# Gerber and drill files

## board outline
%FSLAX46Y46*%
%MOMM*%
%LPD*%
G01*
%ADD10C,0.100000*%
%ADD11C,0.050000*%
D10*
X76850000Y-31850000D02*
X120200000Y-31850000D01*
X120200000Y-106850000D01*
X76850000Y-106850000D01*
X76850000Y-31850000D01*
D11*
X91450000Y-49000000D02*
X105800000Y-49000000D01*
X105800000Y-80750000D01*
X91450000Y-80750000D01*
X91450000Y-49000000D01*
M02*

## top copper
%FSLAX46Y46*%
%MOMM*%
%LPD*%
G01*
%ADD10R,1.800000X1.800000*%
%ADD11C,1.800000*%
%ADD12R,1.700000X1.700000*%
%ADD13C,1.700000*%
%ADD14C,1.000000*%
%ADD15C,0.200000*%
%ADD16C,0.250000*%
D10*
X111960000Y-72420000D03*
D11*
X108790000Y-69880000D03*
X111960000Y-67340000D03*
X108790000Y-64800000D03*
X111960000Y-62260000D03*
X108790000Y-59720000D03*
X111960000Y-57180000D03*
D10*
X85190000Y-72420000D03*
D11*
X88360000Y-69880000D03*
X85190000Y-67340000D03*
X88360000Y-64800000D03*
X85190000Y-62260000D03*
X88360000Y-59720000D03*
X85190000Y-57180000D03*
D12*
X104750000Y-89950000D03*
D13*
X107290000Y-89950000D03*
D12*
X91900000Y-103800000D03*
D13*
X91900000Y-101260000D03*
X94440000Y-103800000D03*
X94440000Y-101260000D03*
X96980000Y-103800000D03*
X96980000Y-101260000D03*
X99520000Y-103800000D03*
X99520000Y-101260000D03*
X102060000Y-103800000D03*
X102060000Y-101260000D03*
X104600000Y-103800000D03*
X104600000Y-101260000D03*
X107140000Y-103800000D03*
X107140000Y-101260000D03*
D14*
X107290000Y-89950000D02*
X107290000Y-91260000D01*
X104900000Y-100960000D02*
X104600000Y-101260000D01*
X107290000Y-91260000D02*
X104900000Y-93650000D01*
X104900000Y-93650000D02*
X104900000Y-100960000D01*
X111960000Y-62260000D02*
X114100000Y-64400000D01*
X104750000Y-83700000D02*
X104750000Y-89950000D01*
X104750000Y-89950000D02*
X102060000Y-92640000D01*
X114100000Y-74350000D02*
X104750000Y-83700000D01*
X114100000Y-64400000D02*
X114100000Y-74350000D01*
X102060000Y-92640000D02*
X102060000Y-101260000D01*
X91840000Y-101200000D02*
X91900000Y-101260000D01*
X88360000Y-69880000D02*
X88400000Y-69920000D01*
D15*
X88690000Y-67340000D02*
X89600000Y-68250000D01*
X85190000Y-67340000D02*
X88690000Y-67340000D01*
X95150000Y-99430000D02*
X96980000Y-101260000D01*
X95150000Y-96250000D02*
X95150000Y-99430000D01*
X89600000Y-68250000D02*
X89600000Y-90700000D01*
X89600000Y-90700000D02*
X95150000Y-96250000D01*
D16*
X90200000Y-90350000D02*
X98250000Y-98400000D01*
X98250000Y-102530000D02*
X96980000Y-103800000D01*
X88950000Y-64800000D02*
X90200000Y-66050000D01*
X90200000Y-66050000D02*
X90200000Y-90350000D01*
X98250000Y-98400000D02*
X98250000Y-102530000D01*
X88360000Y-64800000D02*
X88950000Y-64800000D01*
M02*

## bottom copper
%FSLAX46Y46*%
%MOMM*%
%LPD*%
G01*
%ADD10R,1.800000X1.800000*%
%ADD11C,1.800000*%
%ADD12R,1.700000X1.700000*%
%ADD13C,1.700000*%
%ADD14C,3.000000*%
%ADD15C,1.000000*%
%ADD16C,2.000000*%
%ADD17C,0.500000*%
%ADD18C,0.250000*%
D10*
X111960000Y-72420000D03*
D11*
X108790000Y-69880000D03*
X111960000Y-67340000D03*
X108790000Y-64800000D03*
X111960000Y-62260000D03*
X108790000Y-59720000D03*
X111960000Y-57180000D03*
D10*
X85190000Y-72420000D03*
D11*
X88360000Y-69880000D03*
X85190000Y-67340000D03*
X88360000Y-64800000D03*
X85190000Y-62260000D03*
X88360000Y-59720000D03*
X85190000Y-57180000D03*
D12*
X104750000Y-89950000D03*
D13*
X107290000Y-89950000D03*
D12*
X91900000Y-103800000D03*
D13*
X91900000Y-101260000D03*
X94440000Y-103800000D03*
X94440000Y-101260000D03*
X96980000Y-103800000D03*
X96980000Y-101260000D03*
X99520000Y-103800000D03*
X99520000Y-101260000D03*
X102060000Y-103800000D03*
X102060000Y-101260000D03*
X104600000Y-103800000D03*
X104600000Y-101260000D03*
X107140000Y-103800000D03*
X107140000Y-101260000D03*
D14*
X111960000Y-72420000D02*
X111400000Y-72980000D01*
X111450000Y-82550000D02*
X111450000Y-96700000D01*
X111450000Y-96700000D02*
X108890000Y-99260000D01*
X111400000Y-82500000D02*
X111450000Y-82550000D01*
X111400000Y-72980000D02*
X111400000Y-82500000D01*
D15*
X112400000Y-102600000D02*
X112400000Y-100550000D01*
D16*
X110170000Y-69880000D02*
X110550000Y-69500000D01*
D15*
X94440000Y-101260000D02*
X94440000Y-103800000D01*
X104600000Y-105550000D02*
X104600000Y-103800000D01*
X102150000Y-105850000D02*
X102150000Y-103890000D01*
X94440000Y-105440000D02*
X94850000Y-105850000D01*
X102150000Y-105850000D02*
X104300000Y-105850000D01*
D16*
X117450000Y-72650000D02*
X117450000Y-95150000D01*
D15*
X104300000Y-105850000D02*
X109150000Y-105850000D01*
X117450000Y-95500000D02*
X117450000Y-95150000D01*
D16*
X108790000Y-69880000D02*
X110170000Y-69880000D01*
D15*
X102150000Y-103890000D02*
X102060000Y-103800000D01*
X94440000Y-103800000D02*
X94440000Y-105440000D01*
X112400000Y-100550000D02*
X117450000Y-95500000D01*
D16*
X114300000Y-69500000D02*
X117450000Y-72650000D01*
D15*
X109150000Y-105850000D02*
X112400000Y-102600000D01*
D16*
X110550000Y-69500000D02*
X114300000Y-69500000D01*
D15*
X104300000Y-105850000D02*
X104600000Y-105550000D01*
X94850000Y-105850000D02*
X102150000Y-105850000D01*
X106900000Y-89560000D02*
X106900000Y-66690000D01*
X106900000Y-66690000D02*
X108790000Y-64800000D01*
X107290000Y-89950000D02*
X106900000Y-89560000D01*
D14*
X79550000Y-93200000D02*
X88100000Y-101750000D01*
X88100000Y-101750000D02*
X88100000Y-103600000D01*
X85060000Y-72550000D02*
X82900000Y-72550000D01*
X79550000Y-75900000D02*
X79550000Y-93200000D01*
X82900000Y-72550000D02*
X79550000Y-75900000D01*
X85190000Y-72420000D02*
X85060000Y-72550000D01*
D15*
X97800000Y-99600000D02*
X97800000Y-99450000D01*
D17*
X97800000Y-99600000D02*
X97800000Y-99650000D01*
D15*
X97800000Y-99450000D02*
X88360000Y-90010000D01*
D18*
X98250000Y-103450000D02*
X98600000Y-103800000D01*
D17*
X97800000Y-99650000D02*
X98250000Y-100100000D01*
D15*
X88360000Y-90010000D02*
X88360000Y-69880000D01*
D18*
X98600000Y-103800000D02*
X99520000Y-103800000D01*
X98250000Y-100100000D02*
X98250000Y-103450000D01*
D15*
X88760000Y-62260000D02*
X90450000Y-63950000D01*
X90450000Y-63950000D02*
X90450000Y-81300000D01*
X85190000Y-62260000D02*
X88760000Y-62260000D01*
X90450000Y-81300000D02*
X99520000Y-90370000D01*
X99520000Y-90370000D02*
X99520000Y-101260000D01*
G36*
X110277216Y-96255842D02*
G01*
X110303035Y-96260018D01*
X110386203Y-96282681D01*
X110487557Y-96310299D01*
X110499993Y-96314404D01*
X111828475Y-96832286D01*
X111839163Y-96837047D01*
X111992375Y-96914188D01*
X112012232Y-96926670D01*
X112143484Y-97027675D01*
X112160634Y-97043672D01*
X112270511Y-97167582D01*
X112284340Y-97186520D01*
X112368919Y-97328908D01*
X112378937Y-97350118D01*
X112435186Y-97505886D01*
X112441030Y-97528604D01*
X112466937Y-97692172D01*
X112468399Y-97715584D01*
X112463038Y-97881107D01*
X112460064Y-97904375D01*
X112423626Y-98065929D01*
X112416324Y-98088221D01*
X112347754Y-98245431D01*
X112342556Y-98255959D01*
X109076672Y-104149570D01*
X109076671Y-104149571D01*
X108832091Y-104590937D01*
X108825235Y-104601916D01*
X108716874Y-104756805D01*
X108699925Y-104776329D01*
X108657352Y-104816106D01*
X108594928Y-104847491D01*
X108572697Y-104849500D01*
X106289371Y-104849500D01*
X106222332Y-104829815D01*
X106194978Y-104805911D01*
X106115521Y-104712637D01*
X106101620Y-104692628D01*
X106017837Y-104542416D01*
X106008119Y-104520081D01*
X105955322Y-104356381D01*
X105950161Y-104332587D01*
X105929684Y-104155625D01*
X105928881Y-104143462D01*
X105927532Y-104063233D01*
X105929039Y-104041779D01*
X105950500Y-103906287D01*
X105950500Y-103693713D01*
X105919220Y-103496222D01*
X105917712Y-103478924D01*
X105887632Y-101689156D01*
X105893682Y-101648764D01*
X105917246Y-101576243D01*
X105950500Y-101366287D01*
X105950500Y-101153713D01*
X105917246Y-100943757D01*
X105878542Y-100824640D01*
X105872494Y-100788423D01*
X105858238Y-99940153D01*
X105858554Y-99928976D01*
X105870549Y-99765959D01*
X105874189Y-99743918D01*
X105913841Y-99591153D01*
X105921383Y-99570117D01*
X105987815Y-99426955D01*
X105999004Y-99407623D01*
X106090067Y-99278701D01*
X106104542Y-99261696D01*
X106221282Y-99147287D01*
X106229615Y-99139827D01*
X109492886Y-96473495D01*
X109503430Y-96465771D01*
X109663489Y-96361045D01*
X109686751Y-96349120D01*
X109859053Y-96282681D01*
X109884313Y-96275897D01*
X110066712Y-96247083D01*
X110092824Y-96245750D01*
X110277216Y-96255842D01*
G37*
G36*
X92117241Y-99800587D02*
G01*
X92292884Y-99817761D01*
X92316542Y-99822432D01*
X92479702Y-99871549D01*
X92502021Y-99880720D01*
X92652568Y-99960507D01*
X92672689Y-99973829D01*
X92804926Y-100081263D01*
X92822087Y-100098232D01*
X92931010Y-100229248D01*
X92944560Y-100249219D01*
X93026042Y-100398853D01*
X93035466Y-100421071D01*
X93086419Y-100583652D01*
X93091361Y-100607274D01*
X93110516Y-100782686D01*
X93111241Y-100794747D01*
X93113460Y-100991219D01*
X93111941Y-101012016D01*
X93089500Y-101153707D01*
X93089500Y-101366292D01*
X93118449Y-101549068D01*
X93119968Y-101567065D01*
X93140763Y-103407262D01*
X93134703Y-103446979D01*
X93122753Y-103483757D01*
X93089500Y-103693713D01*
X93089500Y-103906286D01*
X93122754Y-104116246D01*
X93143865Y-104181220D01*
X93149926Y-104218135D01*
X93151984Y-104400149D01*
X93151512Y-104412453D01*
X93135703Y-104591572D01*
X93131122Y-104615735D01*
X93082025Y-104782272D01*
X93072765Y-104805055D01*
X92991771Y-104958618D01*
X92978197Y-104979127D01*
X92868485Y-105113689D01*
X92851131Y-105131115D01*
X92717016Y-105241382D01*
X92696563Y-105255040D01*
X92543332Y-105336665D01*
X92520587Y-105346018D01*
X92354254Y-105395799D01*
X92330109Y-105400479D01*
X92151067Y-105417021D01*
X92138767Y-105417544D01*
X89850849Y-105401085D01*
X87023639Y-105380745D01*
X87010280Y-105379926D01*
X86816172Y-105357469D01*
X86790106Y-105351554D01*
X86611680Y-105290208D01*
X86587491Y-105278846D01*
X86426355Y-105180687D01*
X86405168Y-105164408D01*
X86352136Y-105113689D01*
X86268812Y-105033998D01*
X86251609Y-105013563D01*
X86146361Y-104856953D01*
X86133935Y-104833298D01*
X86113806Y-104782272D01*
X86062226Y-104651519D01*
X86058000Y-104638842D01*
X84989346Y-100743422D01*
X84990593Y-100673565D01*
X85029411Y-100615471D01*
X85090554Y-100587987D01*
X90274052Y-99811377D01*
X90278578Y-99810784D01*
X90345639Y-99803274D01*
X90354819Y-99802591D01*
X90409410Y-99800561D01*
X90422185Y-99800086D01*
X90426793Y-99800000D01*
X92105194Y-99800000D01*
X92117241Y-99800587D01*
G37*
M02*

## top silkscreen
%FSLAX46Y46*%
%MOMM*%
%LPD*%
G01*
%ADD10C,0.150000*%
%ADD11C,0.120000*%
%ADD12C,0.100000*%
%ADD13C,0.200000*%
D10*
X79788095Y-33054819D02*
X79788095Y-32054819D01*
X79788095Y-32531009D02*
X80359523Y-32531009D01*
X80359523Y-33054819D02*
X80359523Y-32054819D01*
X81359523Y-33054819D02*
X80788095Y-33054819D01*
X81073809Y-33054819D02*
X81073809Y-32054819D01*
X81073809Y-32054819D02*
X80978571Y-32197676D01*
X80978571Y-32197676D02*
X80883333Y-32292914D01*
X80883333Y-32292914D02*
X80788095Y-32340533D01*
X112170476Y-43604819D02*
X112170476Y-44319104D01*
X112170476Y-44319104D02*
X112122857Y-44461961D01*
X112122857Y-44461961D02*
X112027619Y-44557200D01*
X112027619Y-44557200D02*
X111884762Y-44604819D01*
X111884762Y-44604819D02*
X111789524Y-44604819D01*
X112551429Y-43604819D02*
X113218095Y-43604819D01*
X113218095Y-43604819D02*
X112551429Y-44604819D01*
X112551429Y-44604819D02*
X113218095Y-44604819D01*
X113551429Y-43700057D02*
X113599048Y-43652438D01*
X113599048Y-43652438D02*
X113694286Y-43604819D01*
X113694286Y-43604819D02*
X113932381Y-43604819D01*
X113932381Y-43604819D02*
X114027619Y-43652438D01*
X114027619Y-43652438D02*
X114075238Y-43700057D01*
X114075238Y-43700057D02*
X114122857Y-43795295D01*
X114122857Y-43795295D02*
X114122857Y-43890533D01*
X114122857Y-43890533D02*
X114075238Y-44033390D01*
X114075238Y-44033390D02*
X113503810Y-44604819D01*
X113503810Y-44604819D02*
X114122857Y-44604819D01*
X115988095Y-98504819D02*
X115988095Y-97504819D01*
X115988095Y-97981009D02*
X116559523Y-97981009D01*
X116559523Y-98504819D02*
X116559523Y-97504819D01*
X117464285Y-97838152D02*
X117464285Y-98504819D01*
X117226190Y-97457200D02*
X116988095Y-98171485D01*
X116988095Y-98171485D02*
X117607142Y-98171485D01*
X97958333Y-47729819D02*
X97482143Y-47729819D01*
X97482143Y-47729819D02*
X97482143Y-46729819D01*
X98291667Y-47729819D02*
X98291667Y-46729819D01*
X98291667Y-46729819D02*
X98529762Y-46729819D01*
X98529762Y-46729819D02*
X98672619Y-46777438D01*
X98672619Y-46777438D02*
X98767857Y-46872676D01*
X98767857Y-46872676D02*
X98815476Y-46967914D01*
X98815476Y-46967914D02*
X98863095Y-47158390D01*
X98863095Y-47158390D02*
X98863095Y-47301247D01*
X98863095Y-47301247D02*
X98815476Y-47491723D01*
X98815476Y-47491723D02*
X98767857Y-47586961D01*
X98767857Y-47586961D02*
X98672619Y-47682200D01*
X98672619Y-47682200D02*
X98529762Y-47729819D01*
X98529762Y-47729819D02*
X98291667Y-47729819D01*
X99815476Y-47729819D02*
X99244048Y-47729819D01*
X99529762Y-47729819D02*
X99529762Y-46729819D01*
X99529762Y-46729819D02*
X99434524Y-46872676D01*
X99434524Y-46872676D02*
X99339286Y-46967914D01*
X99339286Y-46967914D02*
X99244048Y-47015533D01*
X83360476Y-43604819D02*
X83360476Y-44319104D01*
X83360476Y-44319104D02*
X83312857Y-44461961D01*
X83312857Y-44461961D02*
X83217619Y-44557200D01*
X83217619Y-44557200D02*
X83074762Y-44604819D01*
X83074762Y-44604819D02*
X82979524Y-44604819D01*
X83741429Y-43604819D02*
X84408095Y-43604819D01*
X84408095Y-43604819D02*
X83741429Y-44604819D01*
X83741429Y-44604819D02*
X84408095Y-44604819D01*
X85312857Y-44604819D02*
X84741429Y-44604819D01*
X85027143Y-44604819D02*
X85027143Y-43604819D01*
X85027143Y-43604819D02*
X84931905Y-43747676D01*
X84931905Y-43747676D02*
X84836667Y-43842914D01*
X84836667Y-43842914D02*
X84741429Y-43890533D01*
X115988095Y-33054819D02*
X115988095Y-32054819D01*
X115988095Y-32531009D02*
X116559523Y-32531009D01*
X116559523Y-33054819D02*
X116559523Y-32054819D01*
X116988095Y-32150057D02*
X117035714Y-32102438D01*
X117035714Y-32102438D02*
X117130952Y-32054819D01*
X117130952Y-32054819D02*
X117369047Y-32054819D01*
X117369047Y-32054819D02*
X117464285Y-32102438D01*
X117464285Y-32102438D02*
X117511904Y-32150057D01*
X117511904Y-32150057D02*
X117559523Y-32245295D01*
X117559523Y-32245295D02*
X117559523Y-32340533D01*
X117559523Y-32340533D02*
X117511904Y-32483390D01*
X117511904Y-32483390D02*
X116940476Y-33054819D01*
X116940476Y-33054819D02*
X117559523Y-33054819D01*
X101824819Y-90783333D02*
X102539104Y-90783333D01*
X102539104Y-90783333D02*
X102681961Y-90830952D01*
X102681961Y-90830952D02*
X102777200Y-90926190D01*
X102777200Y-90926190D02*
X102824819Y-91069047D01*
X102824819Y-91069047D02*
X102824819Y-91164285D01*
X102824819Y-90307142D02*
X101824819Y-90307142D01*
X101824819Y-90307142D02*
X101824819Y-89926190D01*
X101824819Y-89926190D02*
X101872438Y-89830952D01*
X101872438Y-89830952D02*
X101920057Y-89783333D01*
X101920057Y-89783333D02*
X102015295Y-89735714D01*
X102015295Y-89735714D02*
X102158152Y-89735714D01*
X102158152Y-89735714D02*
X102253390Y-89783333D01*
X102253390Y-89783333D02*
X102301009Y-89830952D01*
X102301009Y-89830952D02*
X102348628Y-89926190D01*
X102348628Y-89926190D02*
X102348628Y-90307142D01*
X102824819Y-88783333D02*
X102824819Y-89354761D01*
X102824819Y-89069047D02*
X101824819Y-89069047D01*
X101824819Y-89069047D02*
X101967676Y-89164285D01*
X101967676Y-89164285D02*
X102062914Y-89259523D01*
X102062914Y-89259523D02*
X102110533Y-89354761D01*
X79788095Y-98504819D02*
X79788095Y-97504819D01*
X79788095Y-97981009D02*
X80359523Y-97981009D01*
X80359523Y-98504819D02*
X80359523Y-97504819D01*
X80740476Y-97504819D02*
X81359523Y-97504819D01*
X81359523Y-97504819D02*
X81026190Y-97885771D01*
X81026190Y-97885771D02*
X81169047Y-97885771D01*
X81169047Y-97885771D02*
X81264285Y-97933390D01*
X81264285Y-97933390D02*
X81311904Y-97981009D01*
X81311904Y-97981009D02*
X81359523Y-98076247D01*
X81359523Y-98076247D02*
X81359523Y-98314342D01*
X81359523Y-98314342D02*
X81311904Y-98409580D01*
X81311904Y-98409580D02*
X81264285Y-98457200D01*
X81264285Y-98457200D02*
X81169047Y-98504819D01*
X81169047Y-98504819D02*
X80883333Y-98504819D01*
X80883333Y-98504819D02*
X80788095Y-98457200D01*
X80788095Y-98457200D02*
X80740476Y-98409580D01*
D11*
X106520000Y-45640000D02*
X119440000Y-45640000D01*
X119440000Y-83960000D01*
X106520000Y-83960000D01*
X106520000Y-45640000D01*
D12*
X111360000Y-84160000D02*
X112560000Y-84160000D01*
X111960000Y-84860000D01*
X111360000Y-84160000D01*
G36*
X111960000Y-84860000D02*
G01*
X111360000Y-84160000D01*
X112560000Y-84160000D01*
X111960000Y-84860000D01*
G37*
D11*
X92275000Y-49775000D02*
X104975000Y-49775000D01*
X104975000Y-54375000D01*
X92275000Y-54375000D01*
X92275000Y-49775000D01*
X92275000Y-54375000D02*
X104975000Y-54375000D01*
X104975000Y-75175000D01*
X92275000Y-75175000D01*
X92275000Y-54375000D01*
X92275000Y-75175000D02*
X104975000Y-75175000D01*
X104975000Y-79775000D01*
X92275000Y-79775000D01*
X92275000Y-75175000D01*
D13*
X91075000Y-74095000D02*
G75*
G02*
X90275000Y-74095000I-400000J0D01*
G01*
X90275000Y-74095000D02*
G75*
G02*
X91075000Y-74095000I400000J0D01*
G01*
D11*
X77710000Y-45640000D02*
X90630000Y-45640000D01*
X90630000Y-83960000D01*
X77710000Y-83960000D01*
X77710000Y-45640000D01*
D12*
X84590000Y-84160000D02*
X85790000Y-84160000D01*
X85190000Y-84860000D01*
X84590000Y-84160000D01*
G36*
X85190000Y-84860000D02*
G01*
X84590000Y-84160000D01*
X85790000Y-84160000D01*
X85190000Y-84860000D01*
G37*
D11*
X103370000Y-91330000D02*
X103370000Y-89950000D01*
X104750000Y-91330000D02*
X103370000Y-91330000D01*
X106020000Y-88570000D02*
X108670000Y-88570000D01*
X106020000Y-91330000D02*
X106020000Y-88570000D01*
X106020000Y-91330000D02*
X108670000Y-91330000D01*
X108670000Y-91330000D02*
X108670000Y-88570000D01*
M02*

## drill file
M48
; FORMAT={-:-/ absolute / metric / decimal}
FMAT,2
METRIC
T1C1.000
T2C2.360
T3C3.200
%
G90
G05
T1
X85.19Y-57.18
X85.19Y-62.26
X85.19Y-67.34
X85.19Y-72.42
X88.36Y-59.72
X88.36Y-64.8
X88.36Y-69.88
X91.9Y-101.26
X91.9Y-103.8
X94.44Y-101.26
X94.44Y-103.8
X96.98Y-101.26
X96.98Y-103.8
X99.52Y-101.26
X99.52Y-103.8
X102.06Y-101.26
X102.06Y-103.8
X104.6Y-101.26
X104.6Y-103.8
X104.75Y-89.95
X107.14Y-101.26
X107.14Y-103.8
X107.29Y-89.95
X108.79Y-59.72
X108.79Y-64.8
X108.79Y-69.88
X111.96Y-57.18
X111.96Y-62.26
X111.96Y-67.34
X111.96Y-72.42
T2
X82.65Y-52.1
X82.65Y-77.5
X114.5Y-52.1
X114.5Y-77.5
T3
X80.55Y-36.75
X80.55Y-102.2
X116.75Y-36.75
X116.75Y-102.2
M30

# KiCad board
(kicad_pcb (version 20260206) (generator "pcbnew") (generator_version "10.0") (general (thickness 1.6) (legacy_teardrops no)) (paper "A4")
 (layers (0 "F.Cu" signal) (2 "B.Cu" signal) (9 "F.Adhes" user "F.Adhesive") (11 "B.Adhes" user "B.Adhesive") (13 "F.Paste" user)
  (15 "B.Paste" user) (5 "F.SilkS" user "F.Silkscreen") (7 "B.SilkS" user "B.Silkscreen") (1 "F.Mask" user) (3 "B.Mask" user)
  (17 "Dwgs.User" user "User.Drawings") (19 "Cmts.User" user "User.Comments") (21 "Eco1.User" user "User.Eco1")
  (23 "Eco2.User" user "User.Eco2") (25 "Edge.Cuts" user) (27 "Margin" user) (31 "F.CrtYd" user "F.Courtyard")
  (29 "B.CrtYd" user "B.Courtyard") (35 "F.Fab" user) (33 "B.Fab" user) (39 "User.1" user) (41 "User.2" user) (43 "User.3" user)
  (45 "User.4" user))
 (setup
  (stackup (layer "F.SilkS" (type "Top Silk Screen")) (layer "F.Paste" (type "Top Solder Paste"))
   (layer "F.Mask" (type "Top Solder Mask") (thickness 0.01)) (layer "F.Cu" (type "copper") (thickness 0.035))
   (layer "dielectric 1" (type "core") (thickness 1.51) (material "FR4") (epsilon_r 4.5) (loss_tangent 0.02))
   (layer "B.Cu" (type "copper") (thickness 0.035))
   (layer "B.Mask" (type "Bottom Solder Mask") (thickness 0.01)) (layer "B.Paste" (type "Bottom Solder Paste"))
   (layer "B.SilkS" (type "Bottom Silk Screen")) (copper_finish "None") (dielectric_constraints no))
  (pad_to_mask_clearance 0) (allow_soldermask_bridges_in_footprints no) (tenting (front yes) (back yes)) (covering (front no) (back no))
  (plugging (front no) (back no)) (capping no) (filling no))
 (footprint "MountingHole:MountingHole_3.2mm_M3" (layer "F.Cu") (at 80.55 36.75)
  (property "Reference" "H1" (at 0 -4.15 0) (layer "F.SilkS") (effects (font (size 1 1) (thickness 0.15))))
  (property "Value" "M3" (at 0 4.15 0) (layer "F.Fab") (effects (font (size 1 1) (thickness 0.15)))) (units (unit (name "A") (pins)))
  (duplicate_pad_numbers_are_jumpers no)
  (pad "" np_thru_hole circle (at 0 0) (size 3.2 3.2) (drill 3.2) (layers "*.Cu" "*.Mask")))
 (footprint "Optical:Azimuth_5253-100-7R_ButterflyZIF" (layer "F.Cu") (at 112.98 64.8)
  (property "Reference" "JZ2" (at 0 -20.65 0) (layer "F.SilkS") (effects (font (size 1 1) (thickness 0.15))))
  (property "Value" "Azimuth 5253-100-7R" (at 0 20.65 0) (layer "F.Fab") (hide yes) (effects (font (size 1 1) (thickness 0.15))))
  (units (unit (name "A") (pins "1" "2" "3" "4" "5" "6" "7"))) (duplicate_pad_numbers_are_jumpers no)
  (fp_rect (start -6.46 -19.16) (end 6.46 19.16) (stroke (width 0.12) (type default)) (fill no) (layer "F.SilkS"))
  (fp_poly (pts (xy -1.62 19.36) (xy -0.42 19.36) (xy -1.02 20.06)) (stroke (width 0.1) (type default)) (fill yes) (layer "F.SilkS"))
  (pad "" np_thru_hole circle (at 1.52 -12.7) (size 2.36 2.36) (drill 2.36) (layers "*.Cu" "*.Mask"))
  (pad "" np_thru_hole circle (at 1.52 12.7) (size 2.36 2.36) (drill 2.36) (layers "*.Cu" "*.Mask"))
  (pad "1" thru_hole rect (at -1.02 7.62) (size 1.8 1.8) (drill 1) (layers "*.Cu" "*.Mask") (remove_unused_layers no) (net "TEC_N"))
  (pad "2" thru_hole circle (at -4.19 5.08) (size 1.8 1.8) (drill 1) (layers "*.Cu" "*.Mask") (remove_unused_layers no) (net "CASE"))
  (pad "3" thru_hole circle (at -1.02 2.54) (size 1.8 1.8) (drill 1) (layers "*.Cu" "*.Mask") (remove_unused_layers no)
   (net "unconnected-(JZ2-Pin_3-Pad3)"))
  (pad "4" thru_hole circle (at -4.19 0) (size 1.8 1.8) (drill 1) (layers "*.Cu" "*.Mask") (remove_unused_layers no) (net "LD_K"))
  (pad "5" thru_hole circle (at -1.02 -2.54) (size 1.8 1.8) (drill 1) (layers "*.Cu" "*.Mask") (remove_unused_layers no) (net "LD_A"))
  (pad "6" thru_hole circle (at -4.19 -5.08) (size 1.8 1.8) (drill 1) (layers "*.Cu" "*.Mask") (remove_unused_layers no)
   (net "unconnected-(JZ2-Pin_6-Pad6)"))
  (pad "7" thru_hole circle (at -1.02 -7.62) (size 1.8 1.8) (drill 1) (layers "*.Cu" "*.Mask") (remove_unused_layers no)
   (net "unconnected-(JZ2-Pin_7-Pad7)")))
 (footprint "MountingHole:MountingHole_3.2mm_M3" (layer "F.Cu") (at 116.75 102.2)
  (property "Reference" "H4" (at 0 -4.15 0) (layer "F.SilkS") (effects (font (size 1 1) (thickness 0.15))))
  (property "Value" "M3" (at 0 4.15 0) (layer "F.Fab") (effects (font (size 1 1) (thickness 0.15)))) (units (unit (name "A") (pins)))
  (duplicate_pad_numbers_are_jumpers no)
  (pad "" np_thru_hole circle (at 0 0) (size 3.2 3.2) (drill 3.2) (layers "*.Cu" "*.Mask")))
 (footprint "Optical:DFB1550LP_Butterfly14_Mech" (layer "F.Cu") (at 98.625 64.775)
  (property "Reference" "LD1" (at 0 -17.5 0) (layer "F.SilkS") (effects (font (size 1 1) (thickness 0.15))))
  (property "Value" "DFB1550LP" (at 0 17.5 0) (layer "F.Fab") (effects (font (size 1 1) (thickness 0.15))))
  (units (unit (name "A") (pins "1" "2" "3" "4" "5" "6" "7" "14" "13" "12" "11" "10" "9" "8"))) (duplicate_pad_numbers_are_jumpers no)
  (fp_rect (start -6.35 -15) (end 6.35 -10.4) (stroke (width 0.12) (type solid)) (fill no) (layer "F.SilkS"))
  (fp_rect (start -6.35 -10.4) (end 6.35 10.4) (stroke (width 0.12) (type solid)) (fill no) (layer "F.SilkS"))
  (fp_rect (start -6.35 10.4) (end 6.35 15) (stroke (width 0.12) (type solid)) (fill no) (layer "F.SilkS"))
  (fp_circle (center -7.95 9.32) (end -7.55 9.32) (stroke (width 0.2) (type solid)) (fill no) (layer "F.SilkS")))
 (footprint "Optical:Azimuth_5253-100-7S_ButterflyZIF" (layer "F.Cu") (at 84.17 64.8)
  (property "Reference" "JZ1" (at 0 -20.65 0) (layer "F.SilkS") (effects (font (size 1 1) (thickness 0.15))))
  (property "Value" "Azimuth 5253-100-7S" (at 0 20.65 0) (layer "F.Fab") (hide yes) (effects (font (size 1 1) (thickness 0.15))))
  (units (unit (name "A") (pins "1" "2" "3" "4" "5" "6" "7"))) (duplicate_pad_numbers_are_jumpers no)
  (fp_rect (start -6.46 -19.16) (end 6.46 19.16) (stroke (width 0.12) (type default)) (fill no) (layer "F.SilkS"))
  (fp_poly (pts (xy 0.42 19.36) (xy 1.62 19.36) (xy 1.02 20.06)) (stroke (width 0.1) (type default)) (fill yes) (layer "F.SilkS"))
  (pad "" np_thru_hole circle (at -1.52 -12.7) (size 2.36 2.36) (drill 2.36) (layers "*.Cu" "*.Mask"))
  (pad "" np_thru_hole circle (at -1.52 12.7) (size 2.36 2.36) (drill 2.36) (layers "*.Cu" "*.Mask"))
  (pad "1" thru_hole rect (at 1.02 7.62) (size 1.8 1.8) (drill 1) (layers "*.Cu" "*.Mask") (remove_unused_layers no) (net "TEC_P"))
  (pad "2" thru_hole circle (at 4.19 5.08) (size 1.8 1.8) (drill 1) (layers "*.Cu" "*.Mask") (remove_unused_layers no) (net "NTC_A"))
  (pad "3" thru_hole circle (at 1.02 2.54) (size 1.8 1.8) (drill 1) (layers "*.Cu" "*.Mask") (remove_unused_layers no) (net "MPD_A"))
  (pad "4" thru_hole circle (at 4.19 0) (size 1.8 1.8) (drill 1) (layers "*.Cu" "*.Mask") (remove_unused_layers no) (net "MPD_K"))
  (pad "5" thru_hole circle (at 1.02 -2.54) (size 1.8 1.8) (drill 1) (layers "*.Cu" "*.Mask") (remove_unused_layers no) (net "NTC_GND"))
  (pad "6" thru_hole circle (at 4.19 -5.08) (size 1.8 1.8) (drill 1) (layers "*.Cu" "*.Mask") (remove_unused_layers no)
   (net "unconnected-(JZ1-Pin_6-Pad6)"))
  (pad "7" thru_hole circle (at 1.02 -7.62) (size 1.8 1.8) (drill 1) (layers "*.Cu" "*.Mask") (remove_unused_layers no)
   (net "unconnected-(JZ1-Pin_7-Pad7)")))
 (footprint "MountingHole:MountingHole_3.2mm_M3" (layer "F.Cu") (at 116.75 36.75)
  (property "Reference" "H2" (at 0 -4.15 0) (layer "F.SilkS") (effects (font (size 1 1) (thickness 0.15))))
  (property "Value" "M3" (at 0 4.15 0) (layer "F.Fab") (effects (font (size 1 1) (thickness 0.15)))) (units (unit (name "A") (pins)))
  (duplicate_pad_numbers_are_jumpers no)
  (pad "" np_thru_hole circle (at 0 0) (size 3.2 3.2) (drill 3.2) (layers "*.Cu" "*.Mask")))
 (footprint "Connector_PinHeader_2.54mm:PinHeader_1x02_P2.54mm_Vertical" (layer "F.Cu") (at 104.75 89.95 90)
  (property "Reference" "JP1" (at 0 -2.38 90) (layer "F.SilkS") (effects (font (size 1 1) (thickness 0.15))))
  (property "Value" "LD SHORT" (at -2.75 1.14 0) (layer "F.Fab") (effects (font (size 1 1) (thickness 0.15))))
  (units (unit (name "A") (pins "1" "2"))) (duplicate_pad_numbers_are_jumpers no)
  (fp_line (start -1.38 -1.38) (end 0 -1.38) (stroke (width 0.12) (type solid)) (layer "F.SilkS"))
  (fp_line (start -1.38 0) (end -1.38 -1.38) (stroke (width 0.12) (type solid)) (layer "F.SilkS"))
  (fp_line (start 1.38 1.27) (end 1.38 3.92) (stroke (width 0.12) (type solid)) (layer "F.SilkS"))
  (fp_line (start -1.38 1.27) (end 1.38 1.27) (stroke (width 0.12) (type solid)) (layer "F.SilkS"))
  (fp_line (start -1.38 1.27) (end -1.38 3.92) (stroke (width 0.12) (type solid)) (layer "F.SilkS"))
  (fp_line (start -1.38 3.92) (end 1.38 3.92) (stroke (width 0.12) (type solid)) (layer "F.SilkS"))
  (pad "1" thru_hole rect (at 0 0 90) (size 1.7 1.7) (drill 1) (layers "*.Cu" "*.Mask") (remove_unused_layers no) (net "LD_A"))
  (pad "2" thru_hole circle (at 0 2.54 90) (size 1.7 1.7) (drill 1) (layers "*.Cu" "*.Mask") (remove_unused_layers no) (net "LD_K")))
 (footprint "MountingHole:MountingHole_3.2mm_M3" (layer "F.Cu") (at 80.55 102.2)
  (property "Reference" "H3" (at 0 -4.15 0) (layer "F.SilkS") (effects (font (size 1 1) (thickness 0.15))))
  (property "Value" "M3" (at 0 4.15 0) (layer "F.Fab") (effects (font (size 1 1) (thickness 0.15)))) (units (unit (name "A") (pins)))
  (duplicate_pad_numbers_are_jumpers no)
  (pad "" np_thru_hole circle (at 0 0) (size 3.2 3.2) (drill 3.2) (layers "*.Cu" "*.Mask")))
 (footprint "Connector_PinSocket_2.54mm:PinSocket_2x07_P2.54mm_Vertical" (layer "B.Cu") (at 91.9 103.8 -90)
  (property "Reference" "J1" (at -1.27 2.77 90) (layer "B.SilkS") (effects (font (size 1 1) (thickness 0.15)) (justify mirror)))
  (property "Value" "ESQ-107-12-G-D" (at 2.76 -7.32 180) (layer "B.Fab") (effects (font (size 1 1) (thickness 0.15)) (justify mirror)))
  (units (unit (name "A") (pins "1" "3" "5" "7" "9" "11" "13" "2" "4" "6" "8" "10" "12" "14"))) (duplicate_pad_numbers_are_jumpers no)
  (pad "1" thru_hole rect (at 0 0 270) (size 1.7 1.7) (drill 1) (layers "*.Cu" "*.Mask") (remove_unused_layers no) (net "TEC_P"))
  (pad "2" thru_hole circle (at -2.54 0 270) (size 1.7 1.7) (drill 1) (layers "*.Cu" "*.Mask") (remove_unused_layers no) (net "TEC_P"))
  (pad "3" thru_hole circle (at 0 -2.54 270) (size 1.7 1.7) (drill 1) (layers "*.Cu" "*.Mask") (remove_unused_layers no) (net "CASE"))
  (pad "4" thru_hole circle (at -2.54 -2.54 270) (size 1.7 1.7) (drill 1) (layers "*.Cu" "*.Mask") (remove_unused_layers no) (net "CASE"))
  (pad "5" thru_hole circle (at 0 -5.08 270) (size 1.7 1.7) (drill 1) (layers "*.Cu" "*.Mask") (remove_unused_layers no) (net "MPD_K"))
  (pad "6" thru_hole circle (at -2.54 -5.08 270) (size 1.7 1.7) (drill 1) (layers "*.Cu" "*.Mask") (remove_unused_layers no) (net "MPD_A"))
  (pad "7" thru_hole circle (at 0 -7.62 270) (size 1.7 1.7) (drill 1) (layers "*.Cu" "*.Mask") (remove_unused_layers no) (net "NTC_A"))
  (pad "8" thru_hole circle (at -2.54 -7.62 270) (size 1.7 1.7) (drill 1) (layers "*.Cu" "*.Mask") (remove_unused_layers no) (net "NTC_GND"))
  (pad "9" thru_hole circle (at 0 -10.16 270) (size 1.7 1.7) (drill 1) (layers "*.Cu" "*.Mask") (remove_unused_layers no) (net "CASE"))
  (pad "10" thru_hole circle (at -2.54 -10.16 270) (size 1.7 1.7) (drill 1) (layers "*.Cu" "*.Mask") (remove_unused_layers no) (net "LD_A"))
  (pad "11" thru_hole circle (at 0 -12.7 270) (size 1.7 1.7) (drill 1) (layers "*.Cu" "*.Mask") (remove_unused_layers no) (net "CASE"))
  (pad "12" thru_hole circle (at -2.54 -12.7 270) (size 1.7 1.7) (drill 1) (layers "*.Cu" "*.Mask") (remove_unused_layers no) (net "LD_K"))
  (pad "13" thru_hole circle (at 0 -15.24 270) (size 1.7 1.7) (drill 1) (layers "*.Cu" "*.Mask") (remove_unused_layers no) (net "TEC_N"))
  (pad "14" thru_hole circle (at -2.54 -15.24 270) (size 1.7 1.7) (drill 1) (layers "*.Cu" "*.Mask") (remove_unused_layers no) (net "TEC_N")))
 (gr_rect (start 76.85 31.85) (end 120.2 106.85) (stroke (width 0.1) (type solid)) (fill no) (layer "Edge.Cuts"))
 (gr_rect (start 91.45 49) (end 105.8 80.75) (stroke (width 0.05) (type default)) (fill no) (layer "Edge.Cuts"))
 (segment (start 111.96 72.42) (end 111.4 72.98) (width 3) (layer "B.Cu") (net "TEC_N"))
 (segment (start 111.45 82.55) (end 111.45 96.7) (width 3) (layer "B.Cu") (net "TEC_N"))
 (segment (start 111.45 96.7) (end 108.89 99.26) (width 3) (layer "B.Cu") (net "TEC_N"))
 (segment (start 111.4 82.5) (end 111.45 82.55) (width 3) (layer "B.Cu") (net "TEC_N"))
 (segment (start 111.4 72.98) (end 111.4 82.5) (width 3) (layer "B.Cu") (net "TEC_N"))
 (segment (start 112.4 102.6) (end 112.4 100.55) (width 1) (layer "B.Cu") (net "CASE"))
 (segment (start 110.17 69.88) (end 110.55 69.5) (width 2) (layer "B.Cu") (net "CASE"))
 (segment (start 94.44 101.26) (end 94.44 103.8) (width 1) (layer "B.Cu") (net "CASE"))
 (segment (start 104.6 105.55) (end 104.6 103.8) (width 1) (layer "B.Cu") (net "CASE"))
 (segment (start 102.15 105.85) (end 102.15 103.89) (width 1) (layer "B.Cu") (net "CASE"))
 (segment (start 94.44 105.44) (end 94.85 105.85) (width 1) (layer "B.Cu") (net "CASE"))
 (segment (start 102.15 105.85) (end 104.3 105.85) (width 1) (layer "B.Cu") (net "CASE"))
 (segment (start 117.45 72.65) (end 117.45 95.15) (width 2) (layer "B.Cu") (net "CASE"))
 (segment (start 104.3 105.85) (end 109.15 105.85) (width 1) (layer "B.Cu") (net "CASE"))
 (segment (start 117.45 95.5) (end 117.45 95.15) (width 1) (layer "B.Cu") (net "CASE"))
 (segment (start 108.79 69.88) (end 110.17 69.88) (width 2) (layer "B.Cu") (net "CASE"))
 (segment (start 102.15 103.89) (end 102.06 103.8) (width 1) (layer "B.Cu") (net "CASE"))
 (segment (start 94.44 103.8) (end 94.44 105.44) (width 1) (layer "B.Cu") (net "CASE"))
 (segment (start 112.4 100.55) (end 117.45 95.5) (width 1) (layer "B.Cu") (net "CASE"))
 (segment (start 114.3 69.5) (end 117.45 72.65) (width 2) (layer "B.Cu") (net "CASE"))
 (segment (start 109.15 105.85) (end 112.4 102.6) (width 1) (layer "B.Cu") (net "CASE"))
 (segment (start 110.55 69.5) (end 114.3 69.5) (width 2) (layer "B.Cu") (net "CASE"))
 (segment (start 104.3 105.85) (end 104.6 105.55) (width 1) (layer "B.Cu") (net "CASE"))
 (segment (start 94.85 105.85) (end 102.15 105.85) (width 1) (layer "B.Cu") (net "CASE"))
 (segment (start 107.29 89.95) (end 107.29 91.26) (width 1) (layer "F.Cu") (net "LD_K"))
 (segment (start 104.9 100.96) (end 104.6 101.26) (width 1) (layer "F.Cu") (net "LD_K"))
 (segment (start 107.29 91.26) (end 104.9 93.65) (width 1) (layer "F.Cu") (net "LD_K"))
 (segment (start 104.9 93.65) (end 104.9 100.96) (width 1) (layer "F.Cu") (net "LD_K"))
 (segment (start 106.9 89.56) (end 106.9 66.69) (width 1) (layer "B.Cu") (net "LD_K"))
 (segment (start 106.9 66.69) (end 108.79 64.8) (width 1) (layer "B.Cu") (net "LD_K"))
 (segment (start 107.29 89.95) (end 106.9 89.56) (width 1) (layer "B.Cu") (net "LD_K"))
 (segment (start 111.96 62.26) (end 114.1 64.4) (width 1) (layer "F.Cu") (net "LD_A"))
 (segment (start 104.75 83.7) (end 104.75 89.95) (width 1) (layer "F.Cu") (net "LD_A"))
 (segment (start 104.75 89.95) (end 102.06 92.64) (width 1) (layer "F.Cu") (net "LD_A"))
 (segment (start 114.1 74.35) (end 104.75 83.7) (width 1) (layer "F.Cu") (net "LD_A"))
 (segment (start 114.1 64.4) (end 114.1 74.35) (width 1) (layer "F.Cu") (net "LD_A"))
 (segment (start 102.06 92.64) (end 102.06 101.26) (width 1) (layer "F.Cu") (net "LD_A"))
 (segment (start 91.84 101.2) (end 91.9 101.26) (width 1) (layer "F.Cu") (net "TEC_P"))
 (segment (start 79.55 93.2) (end 88.1 101.75) (width 3) (layer "B.Cu") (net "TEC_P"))
 (segment (start 88.1 101.75) (end 88.1 103.6) (width 3) (layer "B.Cu") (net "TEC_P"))
 (segment (start 85.06 72.55) (end 82.9 72.55) (width 3) (layer "B.Cu") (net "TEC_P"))
 (segment (start 79.55 75.9) (end 79.55 93.2) (width 3) (layer "B.Cu") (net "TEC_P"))
 (segment (start 82.9 72.55) (end 79.55 75.9) (width 3) (layer "B.Cu") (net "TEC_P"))
 (segment (start 85.19 72.42) (end 85.06 72.55) (width 3) (layer "B.Cu") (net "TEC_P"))
 (segment (start 88.36 69.88) (end 88.4 69.92) (width 1) (layer "F.Cu") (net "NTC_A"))
 (segment (start 97.8 99.6) (end 97.8 99.45) (width 1) (layer "B.Cu") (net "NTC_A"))
 (segment (start 97.8 99.6) (end 97.8 99.65) (width 0.5) (layer "B.Cu") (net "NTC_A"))
 (segment (start 97.8 99.45) (end 88.36 90.01) (width 1) (layer "B.Cu") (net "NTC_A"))
 (segment (start 98.25 103.45) (end 98.6 103.8) (width 0.25) (layer "B.Cu") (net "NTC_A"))
 (segment (start 97.8 99.65) (end 98.25 100.1) (width 0.5) (layer "B.Cu") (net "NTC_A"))
 (segment (start 88.36 90.01) (end 88.36 69.88) (width 1) (layer "B.Cu") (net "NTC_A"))
 (segment (start 98.6 103.8) (end 99.52 103.8) (width 0.25) (layer "B.Cu") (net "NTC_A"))
 (segment (start 98.25 100.1) (end 98.25 103.45) (width 0.25) (layer "B.Cu") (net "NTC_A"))
 (segment (start 88.69 67.34) (end 89.6 68.25) (width 0.2) (layer "F.Cu") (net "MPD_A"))
 (segment (start 85.19 67.34) (end 88.69 67.34) (width 0.2) (layer "F.Cu") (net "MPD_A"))
 (segment (start 95.15 99.43) (end 96.98 101.26) (width 0.2) (layer "F.Cu") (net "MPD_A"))
 (segment (start 95.15 96.25) (end 95.15 99.43) (width 0.2) (layer "F.Cu") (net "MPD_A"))
 (segment (start 89.6 68.25) (end 89.6 90.7) (width 0.2) (layer "F.Cu") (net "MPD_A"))
 (segment (start 89.6 90.7) (end 95.15 96.25) (width 0.2) (layer "F.Cu") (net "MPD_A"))
 (segment (start 90.2 90.35) (end 98.25 98.4) (width 0.25) (layer "F.Cu") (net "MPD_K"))
 (segment (start 98.25 102.53) (end 96.98 103.8) (width 0.25) (layer "F.Cu") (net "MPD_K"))
 (segment (start 88.95 64.8) (end 90.2 66.05) (width 0.25) (layer "F.Cu") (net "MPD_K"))
 (segment (start 90.2 66.05) (end 90.2 90.35) (width 0.25) (layer "F.Cu") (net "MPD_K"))
 (segment (start 98.25 98.4) (end 98.25 102.53) (width 0.25) (layer "F.Cu") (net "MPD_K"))
 (segment (start 88.36 64.8) (end 88.95 64.8) (width 0.25) (layer "F.Cu") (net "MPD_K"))
 (segment (start 88.76 62.26) (end 90.45 63.95) (width 1) (layer "B.Cu") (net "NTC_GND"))
 (segment (start 90.45 63.95) (end 90.45 81.3) (width 1) (layer "B.Cu") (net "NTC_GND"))
 (segment (start 85.19 62.26) (end 88.76 62.26) (width 1) (layer "B.Cu") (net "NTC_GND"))
 (segment (start 90.45 81.3) (end 99.52 90.37) (width 1) (layer "B.Cu") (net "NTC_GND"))
 (segment (start 99.52 90.37) (end 99.52 101.26) (width 1) (layer "B.Cu") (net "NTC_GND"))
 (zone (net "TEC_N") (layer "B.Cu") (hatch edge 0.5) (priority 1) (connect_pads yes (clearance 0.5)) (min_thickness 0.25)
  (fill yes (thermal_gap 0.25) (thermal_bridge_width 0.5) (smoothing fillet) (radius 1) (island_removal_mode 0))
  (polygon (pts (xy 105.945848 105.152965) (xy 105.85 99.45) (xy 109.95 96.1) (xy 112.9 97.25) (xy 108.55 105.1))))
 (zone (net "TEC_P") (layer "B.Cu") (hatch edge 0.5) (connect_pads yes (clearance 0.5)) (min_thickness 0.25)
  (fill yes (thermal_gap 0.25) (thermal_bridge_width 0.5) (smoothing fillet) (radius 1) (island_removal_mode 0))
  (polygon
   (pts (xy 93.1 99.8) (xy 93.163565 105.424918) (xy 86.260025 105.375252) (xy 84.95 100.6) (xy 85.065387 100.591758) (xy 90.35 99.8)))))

